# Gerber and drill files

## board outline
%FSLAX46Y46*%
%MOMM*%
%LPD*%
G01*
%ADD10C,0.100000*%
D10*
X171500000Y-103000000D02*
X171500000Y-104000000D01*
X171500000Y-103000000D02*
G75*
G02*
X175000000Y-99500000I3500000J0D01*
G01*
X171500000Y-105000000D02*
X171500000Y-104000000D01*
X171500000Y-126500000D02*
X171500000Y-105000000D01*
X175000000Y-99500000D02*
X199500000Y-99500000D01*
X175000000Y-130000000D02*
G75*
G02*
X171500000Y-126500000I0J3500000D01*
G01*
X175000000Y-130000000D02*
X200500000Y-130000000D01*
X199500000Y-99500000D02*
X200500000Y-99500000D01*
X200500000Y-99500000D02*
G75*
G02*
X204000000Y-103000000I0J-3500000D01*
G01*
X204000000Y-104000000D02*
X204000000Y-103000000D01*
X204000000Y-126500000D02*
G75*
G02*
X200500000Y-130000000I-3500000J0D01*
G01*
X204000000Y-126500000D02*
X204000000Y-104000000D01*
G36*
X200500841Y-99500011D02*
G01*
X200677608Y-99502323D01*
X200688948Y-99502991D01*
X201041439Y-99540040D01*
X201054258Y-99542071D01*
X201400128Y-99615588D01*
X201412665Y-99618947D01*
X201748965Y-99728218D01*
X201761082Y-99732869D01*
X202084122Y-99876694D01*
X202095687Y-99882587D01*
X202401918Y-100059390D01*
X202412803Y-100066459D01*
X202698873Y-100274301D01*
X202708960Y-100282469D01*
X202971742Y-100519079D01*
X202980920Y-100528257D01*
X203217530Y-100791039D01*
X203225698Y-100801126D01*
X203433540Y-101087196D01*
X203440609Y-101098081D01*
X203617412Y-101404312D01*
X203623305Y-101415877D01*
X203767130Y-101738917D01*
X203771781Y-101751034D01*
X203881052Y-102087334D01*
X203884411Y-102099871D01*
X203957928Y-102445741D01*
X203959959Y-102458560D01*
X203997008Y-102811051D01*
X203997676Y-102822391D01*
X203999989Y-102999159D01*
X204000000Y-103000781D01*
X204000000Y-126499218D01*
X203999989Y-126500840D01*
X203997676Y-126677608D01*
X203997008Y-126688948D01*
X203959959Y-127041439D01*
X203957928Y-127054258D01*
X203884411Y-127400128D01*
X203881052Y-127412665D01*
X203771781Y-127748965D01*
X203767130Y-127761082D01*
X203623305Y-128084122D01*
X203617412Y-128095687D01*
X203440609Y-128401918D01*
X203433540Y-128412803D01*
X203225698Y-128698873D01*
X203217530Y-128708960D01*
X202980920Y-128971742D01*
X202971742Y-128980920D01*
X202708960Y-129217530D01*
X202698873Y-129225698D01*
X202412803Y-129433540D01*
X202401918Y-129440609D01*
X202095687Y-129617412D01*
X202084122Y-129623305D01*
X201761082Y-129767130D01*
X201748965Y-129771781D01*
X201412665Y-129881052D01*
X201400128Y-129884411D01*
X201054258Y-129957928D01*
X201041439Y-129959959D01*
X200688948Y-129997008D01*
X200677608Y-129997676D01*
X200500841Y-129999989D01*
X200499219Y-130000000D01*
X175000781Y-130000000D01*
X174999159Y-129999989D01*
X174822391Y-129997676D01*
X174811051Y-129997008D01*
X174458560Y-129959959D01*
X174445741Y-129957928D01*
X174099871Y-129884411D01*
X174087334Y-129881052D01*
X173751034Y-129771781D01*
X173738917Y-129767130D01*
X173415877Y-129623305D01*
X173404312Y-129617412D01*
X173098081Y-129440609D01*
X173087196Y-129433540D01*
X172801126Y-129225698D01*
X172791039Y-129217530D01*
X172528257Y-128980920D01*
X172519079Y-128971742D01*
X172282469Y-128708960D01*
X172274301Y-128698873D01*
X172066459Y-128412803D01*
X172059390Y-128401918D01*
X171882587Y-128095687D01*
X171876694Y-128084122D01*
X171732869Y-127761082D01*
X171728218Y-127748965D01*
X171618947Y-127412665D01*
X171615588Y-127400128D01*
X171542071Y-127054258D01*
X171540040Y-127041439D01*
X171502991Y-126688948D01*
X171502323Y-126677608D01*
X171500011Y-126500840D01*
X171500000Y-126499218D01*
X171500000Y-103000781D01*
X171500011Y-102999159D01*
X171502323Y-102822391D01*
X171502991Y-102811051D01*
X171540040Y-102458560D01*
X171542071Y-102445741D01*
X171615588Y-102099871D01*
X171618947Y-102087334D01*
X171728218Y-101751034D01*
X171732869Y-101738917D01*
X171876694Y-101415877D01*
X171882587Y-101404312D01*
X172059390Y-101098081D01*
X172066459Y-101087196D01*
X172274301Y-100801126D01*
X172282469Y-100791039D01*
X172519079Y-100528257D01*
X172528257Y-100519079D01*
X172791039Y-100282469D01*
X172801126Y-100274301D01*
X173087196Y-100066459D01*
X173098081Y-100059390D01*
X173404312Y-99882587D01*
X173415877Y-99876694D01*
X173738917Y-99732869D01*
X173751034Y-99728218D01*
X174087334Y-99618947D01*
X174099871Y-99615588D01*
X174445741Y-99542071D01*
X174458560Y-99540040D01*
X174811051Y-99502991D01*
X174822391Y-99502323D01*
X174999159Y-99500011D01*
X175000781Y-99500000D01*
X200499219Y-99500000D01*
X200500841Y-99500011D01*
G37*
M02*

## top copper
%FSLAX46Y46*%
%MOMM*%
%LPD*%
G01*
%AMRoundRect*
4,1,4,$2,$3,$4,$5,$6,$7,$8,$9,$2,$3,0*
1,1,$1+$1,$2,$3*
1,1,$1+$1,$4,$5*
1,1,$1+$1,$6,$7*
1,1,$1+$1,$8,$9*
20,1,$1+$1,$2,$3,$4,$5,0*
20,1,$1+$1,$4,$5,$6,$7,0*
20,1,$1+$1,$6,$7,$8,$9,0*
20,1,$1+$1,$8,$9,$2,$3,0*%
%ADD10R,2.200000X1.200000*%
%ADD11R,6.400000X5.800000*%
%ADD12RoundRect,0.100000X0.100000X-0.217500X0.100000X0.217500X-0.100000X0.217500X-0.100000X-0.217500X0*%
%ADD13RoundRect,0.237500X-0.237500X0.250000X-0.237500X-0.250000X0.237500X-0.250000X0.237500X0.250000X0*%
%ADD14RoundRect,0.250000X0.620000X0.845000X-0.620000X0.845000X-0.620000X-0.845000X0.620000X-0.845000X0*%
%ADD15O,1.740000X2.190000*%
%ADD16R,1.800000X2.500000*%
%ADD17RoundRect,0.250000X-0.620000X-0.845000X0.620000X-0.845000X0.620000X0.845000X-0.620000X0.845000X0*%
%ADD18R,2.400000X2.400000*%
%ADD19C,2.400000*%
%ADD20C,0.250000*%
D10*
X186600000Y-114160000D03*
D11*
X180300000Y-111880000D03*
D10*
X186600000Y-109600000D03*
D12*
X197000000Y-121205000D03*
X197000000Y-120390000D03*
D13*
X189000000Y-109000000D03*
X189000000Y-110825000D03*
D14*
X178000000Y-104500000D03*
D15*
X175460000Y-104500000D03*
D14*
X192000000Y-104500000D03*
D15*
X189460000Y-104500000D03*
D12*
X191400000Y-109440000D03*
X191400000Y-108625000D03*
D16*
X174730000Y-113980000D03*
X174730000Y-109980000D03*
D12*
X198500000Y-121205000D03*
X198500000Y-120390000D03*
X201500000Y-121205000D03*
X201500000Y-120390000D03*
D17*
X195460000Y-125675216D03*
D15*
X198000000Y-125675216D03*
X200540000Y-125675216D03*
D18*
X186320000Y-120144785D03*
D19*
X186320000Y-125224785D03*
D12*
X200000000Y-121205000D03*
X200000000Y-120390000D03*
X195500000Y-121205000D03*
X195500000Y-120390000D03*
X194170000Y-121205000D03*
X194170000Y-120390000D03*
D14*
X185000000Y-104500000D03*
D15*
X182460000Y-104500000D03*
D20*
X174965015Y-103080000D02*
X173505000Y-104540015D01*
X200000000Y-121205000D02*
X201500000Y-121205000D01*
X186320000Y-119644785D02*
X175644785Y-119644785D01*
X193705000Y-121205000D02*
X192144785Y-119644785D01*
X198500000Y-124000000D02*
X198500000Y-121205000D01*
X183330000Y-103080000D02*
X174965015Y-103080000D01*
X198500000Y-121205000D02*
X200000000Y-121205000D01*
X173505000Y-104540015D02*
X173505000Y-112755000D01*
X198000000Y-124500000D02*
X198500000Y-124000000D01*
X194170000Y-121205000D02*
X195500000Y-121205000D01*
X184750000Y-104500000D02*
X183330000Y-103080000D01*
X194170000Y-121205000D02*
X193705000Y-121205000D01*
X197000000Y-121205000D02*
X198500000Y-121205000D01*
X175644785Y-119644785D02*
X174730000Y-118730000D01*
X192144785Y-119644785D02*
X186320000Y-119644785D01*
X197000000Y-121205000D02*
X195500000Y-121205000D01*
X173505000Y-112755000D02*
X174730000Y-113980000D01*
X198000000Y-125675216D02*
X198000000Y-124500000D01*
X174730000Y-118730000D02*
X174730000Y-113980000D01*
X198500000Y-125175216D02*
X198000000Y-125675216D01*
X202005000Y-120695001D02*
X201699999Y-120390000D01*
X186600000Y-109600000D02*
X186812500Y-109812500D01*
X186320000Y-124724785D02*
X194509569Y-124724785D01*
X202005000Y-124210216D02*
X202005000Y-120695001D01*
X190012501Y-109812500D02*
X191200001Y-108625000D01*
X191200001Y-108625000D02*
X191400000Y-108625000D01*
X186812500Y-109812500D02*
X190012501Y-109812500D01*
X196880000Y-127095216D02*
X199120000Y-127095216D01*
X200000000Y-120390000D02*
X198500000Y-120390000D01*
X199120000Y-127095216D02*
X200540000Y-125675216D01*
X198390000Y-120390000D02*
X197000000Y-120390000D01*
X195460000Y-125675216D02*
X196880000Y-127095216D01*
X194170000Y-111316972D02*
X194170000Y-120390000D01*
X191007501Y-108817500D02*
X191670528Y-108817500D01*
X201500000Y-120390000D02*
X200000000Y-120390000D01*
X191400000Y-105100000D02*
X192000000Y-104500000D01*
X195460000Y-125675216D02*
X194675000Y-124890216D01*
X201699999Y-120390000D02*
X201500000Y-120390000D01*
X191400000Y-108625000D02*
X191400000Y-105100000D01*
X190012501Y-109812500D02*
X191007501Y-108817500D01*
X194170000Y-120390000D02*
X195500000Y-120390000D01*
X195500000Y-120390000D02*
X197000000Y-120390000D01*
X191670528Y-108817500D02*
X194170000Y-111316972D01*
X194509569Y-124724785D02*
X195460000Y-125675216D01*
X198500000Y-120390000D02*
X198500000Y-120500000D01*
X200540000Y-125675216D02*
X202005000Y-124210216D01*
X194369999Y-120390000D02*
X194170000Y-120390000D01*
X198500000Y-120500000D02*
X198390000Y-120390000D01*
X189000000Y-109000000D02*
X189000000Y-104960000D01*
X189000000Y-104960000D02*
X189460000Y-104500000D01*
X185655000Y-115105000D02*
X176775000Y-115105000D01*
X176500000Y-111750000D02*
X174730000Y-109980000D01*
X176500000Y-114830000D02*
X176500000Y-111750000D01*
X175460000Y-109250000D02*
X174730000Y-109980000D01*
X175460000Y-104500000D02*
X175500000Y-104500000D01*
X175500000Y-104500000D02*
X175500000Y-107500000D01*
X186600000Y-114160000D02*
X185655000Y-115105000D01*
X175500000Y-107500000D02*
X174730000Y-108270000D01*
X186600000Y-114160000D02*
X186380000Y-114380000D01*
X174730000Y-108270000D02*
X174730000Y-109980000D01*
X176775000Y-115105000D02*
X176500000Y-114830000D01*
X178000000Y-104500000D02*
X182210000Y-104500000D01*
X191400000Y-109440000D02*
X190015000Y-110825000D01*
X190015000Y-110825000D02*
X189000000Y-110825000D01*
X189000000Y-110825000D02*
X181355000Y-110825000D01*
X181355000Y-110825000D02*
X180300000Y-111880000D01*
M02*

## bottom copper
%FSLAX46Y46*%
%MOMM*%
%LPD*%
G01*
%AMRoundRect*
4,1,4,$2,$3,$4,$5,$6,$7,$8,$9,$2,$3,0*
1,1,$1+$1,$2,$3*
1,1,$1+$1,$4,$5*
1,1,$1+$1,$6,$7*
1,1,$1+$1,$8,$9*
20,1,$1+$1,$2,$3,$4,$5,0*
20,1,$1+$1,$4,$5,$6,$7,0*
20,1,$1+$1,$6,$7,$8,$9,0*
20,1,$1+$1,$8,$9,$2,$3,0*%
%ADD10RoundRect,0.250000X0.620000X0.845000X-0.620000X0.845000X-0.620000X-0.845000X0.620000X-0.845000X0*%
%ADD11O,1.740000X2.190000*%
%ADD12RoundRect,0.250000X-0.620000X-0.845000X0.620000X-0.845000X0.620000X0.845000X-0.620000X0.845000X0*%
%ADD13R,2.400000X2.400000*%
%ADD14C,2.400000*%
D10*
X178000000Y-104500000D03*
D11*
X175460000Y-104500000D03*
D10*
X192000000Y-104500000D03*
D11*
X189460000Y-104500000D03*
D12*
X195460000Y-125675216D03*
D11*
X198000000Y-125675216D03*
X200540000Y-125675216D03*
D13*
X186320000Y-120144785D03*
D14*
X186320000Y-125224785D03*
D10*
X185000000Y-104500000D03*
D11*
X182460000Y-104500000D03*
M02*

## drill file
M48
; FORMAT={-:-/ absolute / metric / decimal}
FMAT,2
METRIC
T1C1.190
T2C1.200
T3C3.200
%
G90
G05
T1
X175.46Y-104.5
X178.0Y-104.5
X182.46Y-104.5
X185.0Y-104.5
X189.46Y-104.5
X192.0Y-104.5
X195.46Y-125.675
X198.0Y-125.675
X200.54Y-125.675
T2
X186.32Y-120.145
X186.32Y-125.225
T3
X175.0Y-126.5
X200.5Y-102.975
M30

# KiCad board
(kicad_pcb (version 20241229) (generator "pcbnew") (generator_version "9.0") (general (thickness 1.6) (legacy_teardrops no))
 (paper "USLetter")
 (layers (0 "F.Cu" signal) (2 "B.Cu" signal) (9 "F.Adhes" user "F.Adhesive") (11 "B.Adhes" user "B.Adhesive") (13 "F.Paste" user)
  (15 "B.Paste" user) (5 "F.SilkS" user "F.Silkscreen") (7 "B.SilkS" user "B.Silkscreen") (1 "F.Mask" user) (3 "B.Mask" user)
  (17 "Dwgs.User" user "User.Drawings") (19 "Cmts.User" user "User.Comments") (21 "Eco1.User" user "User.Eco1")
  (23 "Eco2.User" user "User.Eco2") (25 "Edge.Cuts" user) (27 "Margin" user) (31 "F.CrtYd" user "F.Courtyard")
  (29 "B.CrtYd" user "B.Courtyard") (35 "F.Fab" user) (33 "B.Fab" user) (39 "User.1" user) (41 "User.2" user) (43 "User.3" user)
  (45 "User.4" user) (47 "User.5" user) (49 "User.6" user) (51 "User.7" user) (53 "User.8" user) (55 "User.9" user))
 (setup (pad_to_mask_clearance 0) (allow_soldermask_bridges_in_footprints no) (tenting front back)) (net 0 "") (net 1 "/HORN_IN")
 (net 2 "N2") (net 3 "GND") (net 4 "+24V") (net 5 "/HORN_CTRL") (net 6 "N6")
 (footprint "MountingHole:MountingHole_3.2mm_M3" (layer "F.Cu") (at 200.5 102.974874)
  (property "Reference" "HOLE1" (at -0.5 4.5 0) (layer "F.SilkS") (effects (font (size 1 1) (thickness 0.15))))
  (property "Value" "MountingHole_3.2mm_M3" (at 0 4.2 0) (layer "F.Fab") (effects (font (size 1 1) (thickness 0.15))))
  (pad "" np_thru_hole circle (at 0 0) (size 3.2 3.2) (drill 3.2) (layers "*.Cu" "*.Mask")))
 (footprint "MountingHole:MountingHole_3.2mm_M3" (layer "F.Cu") (at 175 126.5)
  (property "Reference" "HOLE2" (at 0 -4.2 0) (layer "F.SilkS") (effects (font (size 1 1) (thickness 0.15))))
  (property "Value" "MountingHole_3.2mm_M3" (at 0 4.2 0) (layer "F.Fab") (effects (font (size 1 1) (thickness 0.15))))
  (pad "" np_thru_hole circle (at 0 0) (size 3.2 3.2) (drill 3.2) (layers "*.Cu" "*.Mask")))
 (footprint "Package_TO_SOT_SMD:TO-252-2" (layer "F.Cu") (at 182.4 111.88 180)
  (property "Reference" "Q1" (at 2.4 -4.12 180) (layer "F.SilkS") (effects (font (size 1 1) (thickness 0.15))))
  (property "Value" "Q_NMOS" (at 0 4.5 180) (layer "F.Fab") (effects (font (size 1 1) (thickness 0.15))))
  (pad "" smd rect (at 0.425 -1.525 180) (size 3.05 2.75) (layers "F.Paste"))
  (pad "" smd rect (at 0.425 1.525 180) (size 3.05 2.75) (layers "F.Paste"))
  (pad "" smd rect (at 3.775 -1.525 180) (size 3.05 2.75) (layers "F.Paste"))
  (pad "" smd rect (at 3.775 1.525 180) (size 3.05 2.75) (layers "F.Paste"))
  (pad "1" smd rect (at -4.2 -2.28 180) (size 2.2 1.2) (layers "F.Cu" "F.Mask" "F.Paste") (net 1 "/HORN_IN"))
  (pad "2" smd rect (at 2.1 0 180) (size 6.4 5.8) (layers "F.Cu" "F.Mask") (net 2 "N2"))
  (pad "3" smd rect (at -4.2 2.28 180) (size 2.2 1.2) (layers "F.Cu" "F.Mask" "F.Paste") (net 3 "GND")))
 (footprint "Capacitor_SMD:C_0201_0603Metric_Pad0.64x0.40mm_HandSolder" (layer "F.Cu") (at 197 120.7975 90)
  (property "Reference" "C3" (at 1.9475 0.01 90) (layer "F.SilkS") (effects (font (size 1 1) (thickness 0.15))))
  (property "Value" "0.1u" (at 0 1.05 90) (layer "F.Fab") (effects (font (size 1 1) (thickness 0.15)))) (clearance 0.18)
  (pad "" smd roundrect (at -0.4325 0 90) (size 0.458 0.36) (layers "F.Paste") (roundrect_rratio 0.25))
  (pad "" smd roundrect (at 0.4325 0 90) (size 0.458 0.36) (layers "F.Paste") (roundrect_rratio 0.25))
  (pad "1" smd roundrect (at -0.4075 0 90) (size 0.635 0.4) (layers "F.Cu" "F.Mask") (roundrect_rratio 0.25) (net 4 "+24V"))
  (pad "2" smd roundrect (at 0.4075 0 90) (size 0.635 0.4) (layers "F.Cu" "F.Mask") (roundrect_rratio 0.25) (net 3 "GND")))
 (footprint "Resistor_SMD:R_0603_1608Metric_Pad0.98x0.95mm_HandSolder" (layer "F.Cu") (at 189 109.9125 -90)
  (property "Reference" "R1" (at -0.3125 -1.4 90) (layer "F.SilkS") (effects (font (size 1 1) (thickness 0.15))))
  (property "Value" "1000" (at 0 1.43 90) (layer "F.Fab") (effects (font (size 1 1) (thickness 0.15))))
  (pad "1" smd roundrect (at -0.9125 0 270) (size 0.975 0.95) (layers "F.Cu" "F.Mask" "F.Paste") (roundrect_rratio 0.25)
   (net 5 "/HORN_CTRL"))
  (pad "2" smd roundrect (at 0.9125 0 270) (size 0.975 0.95) (layers "F.Cu" "F.Mask" "F.Paste") (roundrect_rratio 0.25) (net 2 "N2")))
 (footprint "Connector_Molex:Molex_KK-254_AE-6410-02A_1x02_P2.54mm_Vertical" (layer "F.Cu") (at 178 104.5 180)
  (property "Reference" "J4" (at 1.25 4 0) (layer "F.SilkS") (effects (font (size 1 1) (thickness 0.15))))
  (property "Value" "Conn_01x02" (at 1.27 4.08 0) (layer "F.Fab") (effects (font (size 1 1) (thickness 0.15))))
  (pad "1" thru_hole roundrect (at 0 0 180) (size 1.74 2.19) (drill 1.19) (layers "*.Cu" "*.Mask") (remove_unused_layers no)
   (roundrect_rratio 0.143678) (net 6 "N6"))
  (pad "2" thru_hole oval (at 2.54 0 180) (size 1.74 2.19) (drill 1.19) (layers "*.Cu" "*.Mask") (remove_unused_layers no)
   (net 1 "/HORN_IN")))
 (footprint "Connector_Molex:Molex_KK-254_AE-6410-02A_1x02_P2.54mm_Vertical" (layer "F.Cu") (at 192 104.5 180)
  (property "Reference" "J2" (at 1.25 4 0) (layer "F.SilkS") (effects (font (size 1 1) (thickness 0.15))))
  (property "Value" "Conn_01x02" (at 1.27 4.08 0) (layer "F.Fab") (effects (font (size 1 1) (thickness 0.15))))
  (pad "1" thru_hole roundrect (at 0 0 180) (size 1.74 2.19) (drill 1.19) (layers "*.Cu" "*.Mask") (remove_unused_layers no)
   (roundrect_rratio 0.143678) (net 3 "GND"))
  (pad "2" thru_hole oval (at 2.54 0 180) (size 1.74 2.19) (drill 1.19) (layers "*.Cu" "*.Mask") (remove_unused_layers no)
   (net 5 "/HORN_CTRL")))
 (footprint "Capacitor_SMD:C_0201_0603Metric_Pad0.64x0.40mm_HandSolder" (layer "F.Cu") (at 191.4 109.0325 90)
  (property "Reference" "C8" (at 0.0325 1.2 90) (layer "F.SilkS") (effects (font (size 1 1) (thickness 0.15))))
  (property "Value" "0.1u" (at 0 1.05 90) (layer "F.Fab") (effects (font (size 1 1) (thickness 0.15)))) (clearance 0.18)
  (pad "" smd roundrect (at -0.4325 0 90) (size 0.458 0.36) (layers "F.Paste") (roundrect_rratio 0.25))
  (pad "" smd roundrect (at 0.4325 0 90) (size 0.458 0.36) (layers "F.Paste") (roundrect_rratio 0.25))
  (pad "1" smd roundrect (at -0.4075 0 90) (size 0.635 0.4) (layers "F.Cu" "F.Mask") (roundrect_rratio 0.25) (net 2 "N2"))
  (pad "2" smd roundrect (at 0.4075 0 90) (size 0.635 0.4) (layers "F.Cu" "F.Mask") (roundrect_rratio 0.25) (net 3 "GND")))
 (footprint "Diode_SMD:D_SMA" (layer "F.Cu") (at 174.73 111.98 90)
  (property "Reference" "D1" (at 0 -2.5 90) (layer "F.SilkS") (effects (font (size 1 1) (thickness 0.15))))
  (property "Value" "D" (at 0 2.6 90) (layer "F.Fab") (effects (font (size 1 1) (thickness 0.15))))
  (pad "1" smd rect (at -2 0 90) (size 2.5 1.8) (layers "F.Cu" "F.Mask" "F.Paste") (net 4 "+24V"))
  (pad "2" smd rect (at 2 0 90) (size 2.5 1.8) (layers "F.Cu" "F.Mask" "F.Paste") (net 1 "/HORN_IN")))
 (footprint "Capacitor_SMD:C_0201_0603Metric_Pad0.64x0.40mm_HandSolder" (layer "F.Cu") (at 198.5 120.7975 90)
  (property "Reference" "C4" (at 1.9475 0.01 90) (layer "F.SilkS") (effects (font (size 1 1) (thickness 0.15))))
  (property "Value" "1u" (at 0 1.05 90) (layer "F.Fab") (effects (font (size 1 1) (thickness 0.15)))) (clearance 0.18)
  (pad "" smd roundrect (at -0.4325 0 90) (size 0.458 0.36) (layers "F.Paste") (roundrect_rratio 0.25))
  (pad "" smd roundrect (at 0.4325 0 90) (size 0.458 0.36) (layers "F.Paste") (roundrect_rratio 0.25))
  (pad "1" smd roundrect (at -0.4075 0 90) (size 0.635 0.4) (layers "F.Cu" "F.Mask") (roundrect_rratio 0.25) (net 4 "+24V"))
  (pad "2" smd roundrect (at 0.4075 0 90) (size 0.635 0.4) (layers "F.Cu" "F.Mask") (roundrect_rratio 0.25) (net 3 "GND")))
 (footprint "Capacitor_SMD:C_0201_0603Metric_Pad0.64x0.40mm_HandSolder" (layer "F.Cu") (at 201.5 120.7975 90)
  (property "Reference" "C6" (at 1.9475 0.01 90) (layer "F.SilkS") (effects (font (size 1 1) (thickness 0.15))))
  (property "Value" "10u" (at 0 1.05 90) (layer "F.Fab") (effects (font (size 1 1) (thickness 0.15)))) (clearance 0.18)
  (pad "" smd roundrect (at -0.4325 0 90) (size 0.458 0.36) (layers "F.Paste") (roundrect_rratio 0.25))
  (pad "" smd roundrect (at 0.4325 0 90) (size 0.458 0.36) (layers "F.Paste") (roundrect_rratio 0.25))
  (pad "1" smd roundrect (at -0.4075 0 90) (size 0.635 0.4) (layers "F.Cu" "F.Mask") (roundrect_rratio 0.25) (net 4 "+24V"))
  (pad "2" smd roundrect (at 0.4075 0 90) (size 0.635 0.4) (layers "F.Cu" "F.Mask") (roundrect_rratio 0.25) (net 3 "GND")))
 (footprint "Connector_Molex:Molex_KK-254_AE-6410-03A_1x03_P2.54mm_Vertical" (layer "F.Cu") (at 195.46 125.675216)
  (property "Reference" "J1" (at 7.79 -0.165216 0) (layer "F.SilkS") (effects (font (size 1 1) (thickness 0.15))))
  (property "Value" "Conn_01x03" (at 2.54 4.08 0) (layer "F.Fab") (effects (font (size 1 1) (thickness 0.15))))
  (pad "1" thru_hole roundrect (at 0 0) (size 1.74 2.19) (drill 1.19) (layers "*.Cu" "*.Mask") (remove_unused_layers no)
   (roundrect_rratio 0.143678) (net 3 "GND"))
  (pad "2" thru_hole oval (at 2.54 0) (size 1.74 2.19) (drill 1.19) (layers "*.Cu" "*.Mask") (remove_unused_layers no) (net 4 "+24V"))
  (pad "3" thru_hole oval (at 5.08 0) (size 1.74 2.19) (drill 1.19) (layers "*.Cu" "*.Mask") (remove_unused_layers no) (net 3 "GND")))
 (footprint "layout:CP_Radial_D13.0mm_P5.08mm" (layer "F.Cu") (at 186.32 120.144785 -90)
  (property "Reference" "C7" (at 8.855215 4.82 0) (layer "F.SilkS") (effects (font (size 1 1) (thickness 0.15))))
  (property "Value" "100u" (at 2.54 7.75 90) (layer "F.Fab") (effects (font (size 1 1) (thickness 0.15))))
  (pad "1" thru_hole rect (at 0 0 270) (size 2.4 2.4) (drill 1.2) (layers "*.Cu" "*.Mask") (remove_unused_layers no) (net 4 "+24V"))
  (pad "2" thru_hole circle (at 5.08 0 270) (size 2.4 2.4) (drill 1.2) (layers "*.Cu" "*.Mask") (remove_unused_layers no) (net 3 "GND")))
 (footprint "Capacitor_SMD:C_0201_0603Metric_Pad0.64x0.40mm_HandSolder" (layer "F.Cu") (at 200 120.7975 90)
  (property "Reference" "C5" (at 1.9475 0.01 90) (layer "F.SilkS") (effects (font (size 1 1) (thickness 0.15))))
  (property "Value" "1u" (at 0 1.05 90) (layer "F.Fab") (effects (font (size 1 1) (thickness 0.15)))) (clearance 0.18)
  (pad "" smd roundrect (at -0.4325 0 90) (size 0.458 0.36) (layers "F.Paste") (roundrect_rratio 0.25))
  (pad "" smd roundrect (at 0.4325 0 90) (size 0.458 0.36) (layers "F.Paste") (roundrect_rratio 0.25))
  (pad "1" smd roundrect (at -0.4075 0 90) (size 0.635 0.4) (layers "F.Cu" "F.Mask") (roundrect_rratio 0.25) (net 4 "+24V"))
  (pad "2" smd roundrect (at 0.4075 0 90) (size 0.635 0.4) (layers "F.Cu" "F.Mask") (roundrect_rratio 0.25) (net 3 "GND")))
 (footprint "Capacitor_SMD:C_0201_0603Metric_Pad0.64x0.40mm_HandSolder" (layer "F.Cu") (at 195.5 120.7975 90)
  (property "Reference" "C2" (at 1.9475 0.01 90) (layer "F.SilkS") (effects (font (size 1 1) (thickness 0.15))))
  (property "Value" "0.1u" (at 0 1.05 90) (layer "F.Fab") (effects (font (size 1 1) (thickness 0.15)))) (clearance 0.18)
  (pad "" smd roundrect (at -0.4325 0 90) (size 0.458 0.36) (layers "F.Paste") (roundrect_rratio 0.25))
  (pad "" smd roundrect (at 0.4325 0 90) (size 0.458 0.36) (layers "F.Paste") (roundrect_rratio 0.25))
  (pad "1" smd roundrect (at -0.4075 0 90) (size 0.635 0.4) (layers "F.Cu" "F.Mask") (roundrect_rratio 0.25) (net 4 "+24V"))
  (pad "2" smd roundrect (at 0.4075 0 90) (size 0.635 0.4) (layers "F.Cu" "F.Mask") (roundrect_rratio 0.25) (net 3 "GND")))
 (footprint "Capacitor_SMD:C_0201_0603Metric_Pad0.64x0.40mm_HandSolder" (layer "F.Cu") (at 194.17 120.7975 90)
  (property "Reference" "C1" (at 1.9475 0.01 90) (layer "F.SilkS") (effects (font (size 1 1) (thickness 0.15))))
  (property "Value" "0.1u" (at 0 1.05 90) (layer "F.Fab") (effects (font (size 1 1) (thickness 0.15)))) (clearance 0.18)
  (pad "" smd roundrect (at -0.4325 0 90) (size 0.458 0.36) (layers "F.Paste") (roundrect_rratio 0.25))
  (pad "" smd roundrect (at 0.4325 0 90) (size 0.458 0.36) (layers "F.Paste") (roundrect_rratio 0.25))
  (pad "1" smd roundrect (at -0.4075 0 90) (size 0.635 0.4) (layers "F.Cu" "F.Mask") (roundrect_rratio 0.25) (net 4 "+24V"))
  (pad "2" smd roundrect (at 0.4075 0 90) (size 0.635 0.4) (layers "F.Cu" "F.Mask") (roundrect_rratio 0.25) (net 3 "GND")))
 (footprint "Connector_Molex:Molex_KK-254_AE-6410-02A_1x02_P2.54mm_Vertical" (layer "F.Cu") (at 185 104.5 180)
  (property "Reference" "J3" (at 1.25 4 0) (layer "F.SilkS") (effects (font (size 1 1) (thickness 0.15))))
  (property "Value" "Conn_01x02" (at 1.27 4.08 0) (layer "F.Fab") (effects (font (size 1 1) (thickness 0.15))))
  (pad "1" thru_hole roundrect (at 0 0 180) (size 1.74 2.19) (drill 1.19) (layers "*.Cu" "*.Mask") (remove_unused_layers no)
   (roundrect_rratio 0.143678) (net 4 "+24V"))
  (pad "2" thru_hole oval (at 2.54 0 180) (size 1.74 2.19) (drill 1.19) (layers "*.Cu" "*.Mask") (remove_unused_layers no) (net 6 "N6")))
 (gr_line (start 171.5 103) (end 171.5 104) (stroke (width 0.1) (type default)) (layer "Edge.Cuts"))
 (gr_arc (start 171.5 103) (mid 172.525126 100.525126) (end 175 99.5) (stroke (width 0.1) (type default)) (layer "Edge.Cuts"))
 (gr_line (start 171.5 105) (end 171.5 104) (stroke (width 0.1) (type default)) (layer "Edge.Cuts"))
 (gr_line (start 171.5 126.5) (end 171.5 105) (stroke (width 0.1) (type default)) (layer "Edge.Cuts"))
 (gr_line (start 175 99.5) (end 199.5 99.5) (stroke (width 0.1) (type solid)) (layer "Edge.Cuts"))
 (gr_arc (start 175 130) (mid 172.525126 128.974874) (end 171.5 126.5) (stroke (width 0.1) (type default)) (layer "Edge.Cuts"))
 (gr_line (start 175 130) (end 200.5 130) (stroke (width 0.1) (type default)) (layer "Edge.Cuts"))
 (gr_line (start 199.5 99.5) (end 200.5 99.5) (stroke (width 0.1) (type default)) (layer "Edge.Cuts"))
 (gr_arc (start 200.5 99.5) (mid 202.974874 100.525126) (end 204 103) (stroke (width 0.1) (type default)) (layer "Edge.Cuts"))
 (gr_line (start 204 104) (end 204 103) (stroke (width 0.1) (type default)) (layer "Edge.Cuts"))
 (gr_arc (start 204 126.5) (mid 202.974874 128.974874) (end 200.5 130) (stroke (width 0.1) (type default)) (layer "Edge.Cuts"))
 (gr_line (start 204 126.5) (end 204 104) (stroke (width 0.1) (type default)) (layer "Edge.Cuts"))
 (segment (start 174.965015 103.08) (end 173.505 104.540015) (width 0.25) (layer "F.Cu") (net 4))
 (segment (start 200 121.205) (end 201.5 121.205) (width 0.25) (layer "F.Cu") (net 4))
 (segment (start 186.32 119.644785) (end 175.644785 119.644785) (width 0.25) (layer "F.Cu") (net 4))
 (segment (start 193.705 121.205) (end 192.144785 119.644785) (width 0.25) (layer "F.Cu") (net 4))
 (segment (start 198.5 124) (end 198.5 121.205) (width 0.25) (layer "F.Cu") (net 4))
 (segment (start 183.33 103.08) (end 174.965015 103.08) (width 0.25) (layer "F.Cu") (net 4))
 (segment (start 198.5 121.205) (end 200 121.205) (width 0.25) (layer "F.Cu") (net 4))
 (segment (start 173.505 104.540015) (end 173.505 112.755) (width 0.25) (layer "F.Cu") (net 4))
 (segment (start 198 124.5) (end 198.5 124) (width 0.25) (layer "F.Cu") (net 4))
 (segment (start 194.17 121.205) (end 195.5 121.205) (width 0.25) (layer "F.Cu") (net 4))
 (segment (start 184.75 104.5) (end 183.33 103.08) (width 0.25) (layer "F.Cu") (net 4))
 (segment (start 194.17 121.205) (end 193.705 121.205) (width 0.25) (layer "F.Cu") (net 4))
 (segment (start 197 121.205) (end 198.5 121.205) (width 0.25) (layer "F.Cu") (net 4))
 (segment (start 175.644785 119.644785) (end 174.73 118.73) (width 0.25) (layer "F.Cu") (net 4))
 (segment (start 192.144785 119.644785) (end 186.32 119.644785) (width 0.25) (layer "F.Cu") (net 4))
 (segment (start 197 121.205) (end 195.5 121.205) (width 0.25) (layer "F.Cu") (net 4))
 (segment (start 173.505 112.755) (end 174.73 113.98) (width 0.25) (layer "F.Cu") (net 4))
 (segment (start 198 125.675216) (end 198 124.5) (width 0.25) (layer "F.Cu") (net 4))
 (segment (start 174.73 118.73) (end 174.73 113.98) (width 0.25) (layer "F.Cu") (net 4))
 (segment (start 198.5 125.175216) (end 198 125.675216) (width 0.25) (layer "F.Cu") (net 4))
 (segment (start 202.005 120.695001) (end 201.699999 120.39) (width 0.25) (layer "F.Cu") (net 3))
 (segment (start 186.6 109.6) (end 186.8125 109.8125) (width 0.25) (layer "F.Cu") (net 3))
 (segment (start 186.32 124.724785) (end 194.509569 124.724785) (width 0.25) (layer "F.Cu") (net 3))
 (segment (start 202.005 124.210216) (end 202.005 120.695001) (width 0.25) (layer "F.Cu") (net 3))
 (segment (start 190.012501 109.8125) (end 191.200001 108.625) (width 0.25) (layer "F.Cu") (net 3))
 (segment (start 191.200001 108.625) (end 191.4 108.625) (width 0.25) (layer "F.Cu") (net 3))
 (segment (start 186.8125 109.8125) (end 190.012501 109.8125) (width 0.25) (layer "F.Cu") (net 3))
 (segment (start 196.88 127.095216) (end 199.12 127.095216) (width 0.25) (layer "F.Cu") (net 3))
 (segment (start 200 120.39) (end 198.5 120.39) (width 0.25) (layer "F.Cu") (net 3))
 (segment (start 199.12 127.095216) (end 200.54 125.675216) (width 0.25) (layer "F.Cu") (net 3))
 (segment (start 198.39 120.39) (end 197 120.39) (width 0.25) (layer "F.Cu") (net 3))
 (segment (start 195.46 125.675216) (end 196.88 127.095216) (width 0.25) (layer "F.Cu") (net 3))
 (segment (start 194.17 111.316972) (end 194.17 120.39) (width 0.25) (layer "F.Cu") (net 3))
 (segment (start 191.007501 108.8175) (end 191.670528 108.8175) (width 0.25) (layer "F.Cu") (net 3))
 (segment (start 201.5 120.39) (end 200 120.39) (width 0.25) (layer "F.Cu") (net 3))
 (segment (start 191.4 105.1) (end 192 104.5) (width 0.25) (layer "F.Cu") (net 3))
 (segment (start 195.46 125.675216) (end 194.675 124.890216) (width 0.25) (layer "F.Cu") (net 3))
 (segment (start 201.699999 120.39) (end 201.5 120.39) (width 0.25) (layer "F.Cu") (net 3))
 (segment (start 191.4 108.625) (end 191.4 105.1) (width 0.25) (layer "F.Cu") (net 3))
 (segment (start 190.012501 109.8125) (end 191.007501 108.8175) (width 0.25) (layer "F.Cu") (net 3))
 (segment (start 194.17 120.39) (end 195.5 120.39) (width 0.25) (layer "F.Cu") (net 3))
 (segment (start 195.5 120.39) (end 197 120.39) (width 0.25) (layer "F.Cu") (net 3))
 (segment (start 191.670528 108.8175) (end 194.17 111.316972) (width 0.25) (layer "F.Cu") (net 3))
 (segment (start 194.509569 124.724785) (end 195.46 125.675216) (width 0.25) (layer "F.Cu") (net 3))
 (segment (start 198.5 120.39) (end 198.5 120.5) (width 0.25) (layer "F.Cu") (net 3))
 (segment (start 200.54 125.675216) (end 202.005 124.210216) (width 0.25) (layer "F.Cu") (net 3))
 (segment (start 194.369999 120.39) (end 194.17 120.39) (width 0.25) (layer "F.Cu") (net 3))
 (segment (start 198.5 120.5) (end 198.39 120.39) (width 0.25) (layer "F.Cu") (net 3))
 (segment (start 189 109) (end 189 104.96) (width 0.25) (layer "F.Cu") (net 5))
 (segment (start 189 104.96) (end 189.46 104.5) (width 0.25) (layer "F.Cu") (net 5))
 (segment (start 185.655 115.105) (end 176.775 115.105) (width 0.25) (layer "F.Cu") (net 1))
 (segment (start 176.5 111.75) (end 174.73 109.98) (width 0.25) (layer "F.Cu") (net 1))
 (segment (start 176.5 114.83) (end 176.5 111.75) (width 0.25) (layer "F.Cu") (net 1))
 (segment (start 175.46 109.25) (end 174.73 109.98) (width 0.25) (layer "F.Cu") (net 1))
 (segment (start 175.46 104.5) (end 175.5 104.5) (width 0.25) (layer "F.Cu") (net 1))
 (segment (start 175.5 104.5) (end 175.5 107.5) (width 0.25) (layer "F.Cu") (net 1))
 (segment (start 186.6 114.16) (end 185.655 115.105) (width 0.25) (layer "F.Cu") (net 1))
 (segment (start 175.5 107.5) (end 174.73 108.27) (width 0.25) (layer "F.Cu") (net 1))
 (segment (start 186.6 114.16) (end 186.38 114.38) (width 0.25) (layer "F.Cu") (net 1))
 (segment (start 174.73 108.27) (end 174.73 109.98) (width 0.25) (layer "F.Cu") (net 1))
 (segment (start 176.775 115.105) (end 176.5 114.83) (width 0.25) (layer "F.Cu") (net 1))
 (segment (start 178 104.5) (end 182.21 104.5) (width 0.25) (layer "F.Cu") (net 6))
 (segment (start 191.4 109.44) (end 190.015 110.825) (width 0.25) (layer "F.Cu") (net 2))
 (segment (start 190.015 110.825) (end 189 110.825) (width 0.25) (layer "F.Cu") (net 2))
 (segment (start 189 110.825) (end 181.355 110.825) (width 0.25) (layer "F.Cu") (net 2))
 (segment (start 181.355 110.825) (end 180.3 111.88) (width 0.25) (layer "F.Cu") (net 2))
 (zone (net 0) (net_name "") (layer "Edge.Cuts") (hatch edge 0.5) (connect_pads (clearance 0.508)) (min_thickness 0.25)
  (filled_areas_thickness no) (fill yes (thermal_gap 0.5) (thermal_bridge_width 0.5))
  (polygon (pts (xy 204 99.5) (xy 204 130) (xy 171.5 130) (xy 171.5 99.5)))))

